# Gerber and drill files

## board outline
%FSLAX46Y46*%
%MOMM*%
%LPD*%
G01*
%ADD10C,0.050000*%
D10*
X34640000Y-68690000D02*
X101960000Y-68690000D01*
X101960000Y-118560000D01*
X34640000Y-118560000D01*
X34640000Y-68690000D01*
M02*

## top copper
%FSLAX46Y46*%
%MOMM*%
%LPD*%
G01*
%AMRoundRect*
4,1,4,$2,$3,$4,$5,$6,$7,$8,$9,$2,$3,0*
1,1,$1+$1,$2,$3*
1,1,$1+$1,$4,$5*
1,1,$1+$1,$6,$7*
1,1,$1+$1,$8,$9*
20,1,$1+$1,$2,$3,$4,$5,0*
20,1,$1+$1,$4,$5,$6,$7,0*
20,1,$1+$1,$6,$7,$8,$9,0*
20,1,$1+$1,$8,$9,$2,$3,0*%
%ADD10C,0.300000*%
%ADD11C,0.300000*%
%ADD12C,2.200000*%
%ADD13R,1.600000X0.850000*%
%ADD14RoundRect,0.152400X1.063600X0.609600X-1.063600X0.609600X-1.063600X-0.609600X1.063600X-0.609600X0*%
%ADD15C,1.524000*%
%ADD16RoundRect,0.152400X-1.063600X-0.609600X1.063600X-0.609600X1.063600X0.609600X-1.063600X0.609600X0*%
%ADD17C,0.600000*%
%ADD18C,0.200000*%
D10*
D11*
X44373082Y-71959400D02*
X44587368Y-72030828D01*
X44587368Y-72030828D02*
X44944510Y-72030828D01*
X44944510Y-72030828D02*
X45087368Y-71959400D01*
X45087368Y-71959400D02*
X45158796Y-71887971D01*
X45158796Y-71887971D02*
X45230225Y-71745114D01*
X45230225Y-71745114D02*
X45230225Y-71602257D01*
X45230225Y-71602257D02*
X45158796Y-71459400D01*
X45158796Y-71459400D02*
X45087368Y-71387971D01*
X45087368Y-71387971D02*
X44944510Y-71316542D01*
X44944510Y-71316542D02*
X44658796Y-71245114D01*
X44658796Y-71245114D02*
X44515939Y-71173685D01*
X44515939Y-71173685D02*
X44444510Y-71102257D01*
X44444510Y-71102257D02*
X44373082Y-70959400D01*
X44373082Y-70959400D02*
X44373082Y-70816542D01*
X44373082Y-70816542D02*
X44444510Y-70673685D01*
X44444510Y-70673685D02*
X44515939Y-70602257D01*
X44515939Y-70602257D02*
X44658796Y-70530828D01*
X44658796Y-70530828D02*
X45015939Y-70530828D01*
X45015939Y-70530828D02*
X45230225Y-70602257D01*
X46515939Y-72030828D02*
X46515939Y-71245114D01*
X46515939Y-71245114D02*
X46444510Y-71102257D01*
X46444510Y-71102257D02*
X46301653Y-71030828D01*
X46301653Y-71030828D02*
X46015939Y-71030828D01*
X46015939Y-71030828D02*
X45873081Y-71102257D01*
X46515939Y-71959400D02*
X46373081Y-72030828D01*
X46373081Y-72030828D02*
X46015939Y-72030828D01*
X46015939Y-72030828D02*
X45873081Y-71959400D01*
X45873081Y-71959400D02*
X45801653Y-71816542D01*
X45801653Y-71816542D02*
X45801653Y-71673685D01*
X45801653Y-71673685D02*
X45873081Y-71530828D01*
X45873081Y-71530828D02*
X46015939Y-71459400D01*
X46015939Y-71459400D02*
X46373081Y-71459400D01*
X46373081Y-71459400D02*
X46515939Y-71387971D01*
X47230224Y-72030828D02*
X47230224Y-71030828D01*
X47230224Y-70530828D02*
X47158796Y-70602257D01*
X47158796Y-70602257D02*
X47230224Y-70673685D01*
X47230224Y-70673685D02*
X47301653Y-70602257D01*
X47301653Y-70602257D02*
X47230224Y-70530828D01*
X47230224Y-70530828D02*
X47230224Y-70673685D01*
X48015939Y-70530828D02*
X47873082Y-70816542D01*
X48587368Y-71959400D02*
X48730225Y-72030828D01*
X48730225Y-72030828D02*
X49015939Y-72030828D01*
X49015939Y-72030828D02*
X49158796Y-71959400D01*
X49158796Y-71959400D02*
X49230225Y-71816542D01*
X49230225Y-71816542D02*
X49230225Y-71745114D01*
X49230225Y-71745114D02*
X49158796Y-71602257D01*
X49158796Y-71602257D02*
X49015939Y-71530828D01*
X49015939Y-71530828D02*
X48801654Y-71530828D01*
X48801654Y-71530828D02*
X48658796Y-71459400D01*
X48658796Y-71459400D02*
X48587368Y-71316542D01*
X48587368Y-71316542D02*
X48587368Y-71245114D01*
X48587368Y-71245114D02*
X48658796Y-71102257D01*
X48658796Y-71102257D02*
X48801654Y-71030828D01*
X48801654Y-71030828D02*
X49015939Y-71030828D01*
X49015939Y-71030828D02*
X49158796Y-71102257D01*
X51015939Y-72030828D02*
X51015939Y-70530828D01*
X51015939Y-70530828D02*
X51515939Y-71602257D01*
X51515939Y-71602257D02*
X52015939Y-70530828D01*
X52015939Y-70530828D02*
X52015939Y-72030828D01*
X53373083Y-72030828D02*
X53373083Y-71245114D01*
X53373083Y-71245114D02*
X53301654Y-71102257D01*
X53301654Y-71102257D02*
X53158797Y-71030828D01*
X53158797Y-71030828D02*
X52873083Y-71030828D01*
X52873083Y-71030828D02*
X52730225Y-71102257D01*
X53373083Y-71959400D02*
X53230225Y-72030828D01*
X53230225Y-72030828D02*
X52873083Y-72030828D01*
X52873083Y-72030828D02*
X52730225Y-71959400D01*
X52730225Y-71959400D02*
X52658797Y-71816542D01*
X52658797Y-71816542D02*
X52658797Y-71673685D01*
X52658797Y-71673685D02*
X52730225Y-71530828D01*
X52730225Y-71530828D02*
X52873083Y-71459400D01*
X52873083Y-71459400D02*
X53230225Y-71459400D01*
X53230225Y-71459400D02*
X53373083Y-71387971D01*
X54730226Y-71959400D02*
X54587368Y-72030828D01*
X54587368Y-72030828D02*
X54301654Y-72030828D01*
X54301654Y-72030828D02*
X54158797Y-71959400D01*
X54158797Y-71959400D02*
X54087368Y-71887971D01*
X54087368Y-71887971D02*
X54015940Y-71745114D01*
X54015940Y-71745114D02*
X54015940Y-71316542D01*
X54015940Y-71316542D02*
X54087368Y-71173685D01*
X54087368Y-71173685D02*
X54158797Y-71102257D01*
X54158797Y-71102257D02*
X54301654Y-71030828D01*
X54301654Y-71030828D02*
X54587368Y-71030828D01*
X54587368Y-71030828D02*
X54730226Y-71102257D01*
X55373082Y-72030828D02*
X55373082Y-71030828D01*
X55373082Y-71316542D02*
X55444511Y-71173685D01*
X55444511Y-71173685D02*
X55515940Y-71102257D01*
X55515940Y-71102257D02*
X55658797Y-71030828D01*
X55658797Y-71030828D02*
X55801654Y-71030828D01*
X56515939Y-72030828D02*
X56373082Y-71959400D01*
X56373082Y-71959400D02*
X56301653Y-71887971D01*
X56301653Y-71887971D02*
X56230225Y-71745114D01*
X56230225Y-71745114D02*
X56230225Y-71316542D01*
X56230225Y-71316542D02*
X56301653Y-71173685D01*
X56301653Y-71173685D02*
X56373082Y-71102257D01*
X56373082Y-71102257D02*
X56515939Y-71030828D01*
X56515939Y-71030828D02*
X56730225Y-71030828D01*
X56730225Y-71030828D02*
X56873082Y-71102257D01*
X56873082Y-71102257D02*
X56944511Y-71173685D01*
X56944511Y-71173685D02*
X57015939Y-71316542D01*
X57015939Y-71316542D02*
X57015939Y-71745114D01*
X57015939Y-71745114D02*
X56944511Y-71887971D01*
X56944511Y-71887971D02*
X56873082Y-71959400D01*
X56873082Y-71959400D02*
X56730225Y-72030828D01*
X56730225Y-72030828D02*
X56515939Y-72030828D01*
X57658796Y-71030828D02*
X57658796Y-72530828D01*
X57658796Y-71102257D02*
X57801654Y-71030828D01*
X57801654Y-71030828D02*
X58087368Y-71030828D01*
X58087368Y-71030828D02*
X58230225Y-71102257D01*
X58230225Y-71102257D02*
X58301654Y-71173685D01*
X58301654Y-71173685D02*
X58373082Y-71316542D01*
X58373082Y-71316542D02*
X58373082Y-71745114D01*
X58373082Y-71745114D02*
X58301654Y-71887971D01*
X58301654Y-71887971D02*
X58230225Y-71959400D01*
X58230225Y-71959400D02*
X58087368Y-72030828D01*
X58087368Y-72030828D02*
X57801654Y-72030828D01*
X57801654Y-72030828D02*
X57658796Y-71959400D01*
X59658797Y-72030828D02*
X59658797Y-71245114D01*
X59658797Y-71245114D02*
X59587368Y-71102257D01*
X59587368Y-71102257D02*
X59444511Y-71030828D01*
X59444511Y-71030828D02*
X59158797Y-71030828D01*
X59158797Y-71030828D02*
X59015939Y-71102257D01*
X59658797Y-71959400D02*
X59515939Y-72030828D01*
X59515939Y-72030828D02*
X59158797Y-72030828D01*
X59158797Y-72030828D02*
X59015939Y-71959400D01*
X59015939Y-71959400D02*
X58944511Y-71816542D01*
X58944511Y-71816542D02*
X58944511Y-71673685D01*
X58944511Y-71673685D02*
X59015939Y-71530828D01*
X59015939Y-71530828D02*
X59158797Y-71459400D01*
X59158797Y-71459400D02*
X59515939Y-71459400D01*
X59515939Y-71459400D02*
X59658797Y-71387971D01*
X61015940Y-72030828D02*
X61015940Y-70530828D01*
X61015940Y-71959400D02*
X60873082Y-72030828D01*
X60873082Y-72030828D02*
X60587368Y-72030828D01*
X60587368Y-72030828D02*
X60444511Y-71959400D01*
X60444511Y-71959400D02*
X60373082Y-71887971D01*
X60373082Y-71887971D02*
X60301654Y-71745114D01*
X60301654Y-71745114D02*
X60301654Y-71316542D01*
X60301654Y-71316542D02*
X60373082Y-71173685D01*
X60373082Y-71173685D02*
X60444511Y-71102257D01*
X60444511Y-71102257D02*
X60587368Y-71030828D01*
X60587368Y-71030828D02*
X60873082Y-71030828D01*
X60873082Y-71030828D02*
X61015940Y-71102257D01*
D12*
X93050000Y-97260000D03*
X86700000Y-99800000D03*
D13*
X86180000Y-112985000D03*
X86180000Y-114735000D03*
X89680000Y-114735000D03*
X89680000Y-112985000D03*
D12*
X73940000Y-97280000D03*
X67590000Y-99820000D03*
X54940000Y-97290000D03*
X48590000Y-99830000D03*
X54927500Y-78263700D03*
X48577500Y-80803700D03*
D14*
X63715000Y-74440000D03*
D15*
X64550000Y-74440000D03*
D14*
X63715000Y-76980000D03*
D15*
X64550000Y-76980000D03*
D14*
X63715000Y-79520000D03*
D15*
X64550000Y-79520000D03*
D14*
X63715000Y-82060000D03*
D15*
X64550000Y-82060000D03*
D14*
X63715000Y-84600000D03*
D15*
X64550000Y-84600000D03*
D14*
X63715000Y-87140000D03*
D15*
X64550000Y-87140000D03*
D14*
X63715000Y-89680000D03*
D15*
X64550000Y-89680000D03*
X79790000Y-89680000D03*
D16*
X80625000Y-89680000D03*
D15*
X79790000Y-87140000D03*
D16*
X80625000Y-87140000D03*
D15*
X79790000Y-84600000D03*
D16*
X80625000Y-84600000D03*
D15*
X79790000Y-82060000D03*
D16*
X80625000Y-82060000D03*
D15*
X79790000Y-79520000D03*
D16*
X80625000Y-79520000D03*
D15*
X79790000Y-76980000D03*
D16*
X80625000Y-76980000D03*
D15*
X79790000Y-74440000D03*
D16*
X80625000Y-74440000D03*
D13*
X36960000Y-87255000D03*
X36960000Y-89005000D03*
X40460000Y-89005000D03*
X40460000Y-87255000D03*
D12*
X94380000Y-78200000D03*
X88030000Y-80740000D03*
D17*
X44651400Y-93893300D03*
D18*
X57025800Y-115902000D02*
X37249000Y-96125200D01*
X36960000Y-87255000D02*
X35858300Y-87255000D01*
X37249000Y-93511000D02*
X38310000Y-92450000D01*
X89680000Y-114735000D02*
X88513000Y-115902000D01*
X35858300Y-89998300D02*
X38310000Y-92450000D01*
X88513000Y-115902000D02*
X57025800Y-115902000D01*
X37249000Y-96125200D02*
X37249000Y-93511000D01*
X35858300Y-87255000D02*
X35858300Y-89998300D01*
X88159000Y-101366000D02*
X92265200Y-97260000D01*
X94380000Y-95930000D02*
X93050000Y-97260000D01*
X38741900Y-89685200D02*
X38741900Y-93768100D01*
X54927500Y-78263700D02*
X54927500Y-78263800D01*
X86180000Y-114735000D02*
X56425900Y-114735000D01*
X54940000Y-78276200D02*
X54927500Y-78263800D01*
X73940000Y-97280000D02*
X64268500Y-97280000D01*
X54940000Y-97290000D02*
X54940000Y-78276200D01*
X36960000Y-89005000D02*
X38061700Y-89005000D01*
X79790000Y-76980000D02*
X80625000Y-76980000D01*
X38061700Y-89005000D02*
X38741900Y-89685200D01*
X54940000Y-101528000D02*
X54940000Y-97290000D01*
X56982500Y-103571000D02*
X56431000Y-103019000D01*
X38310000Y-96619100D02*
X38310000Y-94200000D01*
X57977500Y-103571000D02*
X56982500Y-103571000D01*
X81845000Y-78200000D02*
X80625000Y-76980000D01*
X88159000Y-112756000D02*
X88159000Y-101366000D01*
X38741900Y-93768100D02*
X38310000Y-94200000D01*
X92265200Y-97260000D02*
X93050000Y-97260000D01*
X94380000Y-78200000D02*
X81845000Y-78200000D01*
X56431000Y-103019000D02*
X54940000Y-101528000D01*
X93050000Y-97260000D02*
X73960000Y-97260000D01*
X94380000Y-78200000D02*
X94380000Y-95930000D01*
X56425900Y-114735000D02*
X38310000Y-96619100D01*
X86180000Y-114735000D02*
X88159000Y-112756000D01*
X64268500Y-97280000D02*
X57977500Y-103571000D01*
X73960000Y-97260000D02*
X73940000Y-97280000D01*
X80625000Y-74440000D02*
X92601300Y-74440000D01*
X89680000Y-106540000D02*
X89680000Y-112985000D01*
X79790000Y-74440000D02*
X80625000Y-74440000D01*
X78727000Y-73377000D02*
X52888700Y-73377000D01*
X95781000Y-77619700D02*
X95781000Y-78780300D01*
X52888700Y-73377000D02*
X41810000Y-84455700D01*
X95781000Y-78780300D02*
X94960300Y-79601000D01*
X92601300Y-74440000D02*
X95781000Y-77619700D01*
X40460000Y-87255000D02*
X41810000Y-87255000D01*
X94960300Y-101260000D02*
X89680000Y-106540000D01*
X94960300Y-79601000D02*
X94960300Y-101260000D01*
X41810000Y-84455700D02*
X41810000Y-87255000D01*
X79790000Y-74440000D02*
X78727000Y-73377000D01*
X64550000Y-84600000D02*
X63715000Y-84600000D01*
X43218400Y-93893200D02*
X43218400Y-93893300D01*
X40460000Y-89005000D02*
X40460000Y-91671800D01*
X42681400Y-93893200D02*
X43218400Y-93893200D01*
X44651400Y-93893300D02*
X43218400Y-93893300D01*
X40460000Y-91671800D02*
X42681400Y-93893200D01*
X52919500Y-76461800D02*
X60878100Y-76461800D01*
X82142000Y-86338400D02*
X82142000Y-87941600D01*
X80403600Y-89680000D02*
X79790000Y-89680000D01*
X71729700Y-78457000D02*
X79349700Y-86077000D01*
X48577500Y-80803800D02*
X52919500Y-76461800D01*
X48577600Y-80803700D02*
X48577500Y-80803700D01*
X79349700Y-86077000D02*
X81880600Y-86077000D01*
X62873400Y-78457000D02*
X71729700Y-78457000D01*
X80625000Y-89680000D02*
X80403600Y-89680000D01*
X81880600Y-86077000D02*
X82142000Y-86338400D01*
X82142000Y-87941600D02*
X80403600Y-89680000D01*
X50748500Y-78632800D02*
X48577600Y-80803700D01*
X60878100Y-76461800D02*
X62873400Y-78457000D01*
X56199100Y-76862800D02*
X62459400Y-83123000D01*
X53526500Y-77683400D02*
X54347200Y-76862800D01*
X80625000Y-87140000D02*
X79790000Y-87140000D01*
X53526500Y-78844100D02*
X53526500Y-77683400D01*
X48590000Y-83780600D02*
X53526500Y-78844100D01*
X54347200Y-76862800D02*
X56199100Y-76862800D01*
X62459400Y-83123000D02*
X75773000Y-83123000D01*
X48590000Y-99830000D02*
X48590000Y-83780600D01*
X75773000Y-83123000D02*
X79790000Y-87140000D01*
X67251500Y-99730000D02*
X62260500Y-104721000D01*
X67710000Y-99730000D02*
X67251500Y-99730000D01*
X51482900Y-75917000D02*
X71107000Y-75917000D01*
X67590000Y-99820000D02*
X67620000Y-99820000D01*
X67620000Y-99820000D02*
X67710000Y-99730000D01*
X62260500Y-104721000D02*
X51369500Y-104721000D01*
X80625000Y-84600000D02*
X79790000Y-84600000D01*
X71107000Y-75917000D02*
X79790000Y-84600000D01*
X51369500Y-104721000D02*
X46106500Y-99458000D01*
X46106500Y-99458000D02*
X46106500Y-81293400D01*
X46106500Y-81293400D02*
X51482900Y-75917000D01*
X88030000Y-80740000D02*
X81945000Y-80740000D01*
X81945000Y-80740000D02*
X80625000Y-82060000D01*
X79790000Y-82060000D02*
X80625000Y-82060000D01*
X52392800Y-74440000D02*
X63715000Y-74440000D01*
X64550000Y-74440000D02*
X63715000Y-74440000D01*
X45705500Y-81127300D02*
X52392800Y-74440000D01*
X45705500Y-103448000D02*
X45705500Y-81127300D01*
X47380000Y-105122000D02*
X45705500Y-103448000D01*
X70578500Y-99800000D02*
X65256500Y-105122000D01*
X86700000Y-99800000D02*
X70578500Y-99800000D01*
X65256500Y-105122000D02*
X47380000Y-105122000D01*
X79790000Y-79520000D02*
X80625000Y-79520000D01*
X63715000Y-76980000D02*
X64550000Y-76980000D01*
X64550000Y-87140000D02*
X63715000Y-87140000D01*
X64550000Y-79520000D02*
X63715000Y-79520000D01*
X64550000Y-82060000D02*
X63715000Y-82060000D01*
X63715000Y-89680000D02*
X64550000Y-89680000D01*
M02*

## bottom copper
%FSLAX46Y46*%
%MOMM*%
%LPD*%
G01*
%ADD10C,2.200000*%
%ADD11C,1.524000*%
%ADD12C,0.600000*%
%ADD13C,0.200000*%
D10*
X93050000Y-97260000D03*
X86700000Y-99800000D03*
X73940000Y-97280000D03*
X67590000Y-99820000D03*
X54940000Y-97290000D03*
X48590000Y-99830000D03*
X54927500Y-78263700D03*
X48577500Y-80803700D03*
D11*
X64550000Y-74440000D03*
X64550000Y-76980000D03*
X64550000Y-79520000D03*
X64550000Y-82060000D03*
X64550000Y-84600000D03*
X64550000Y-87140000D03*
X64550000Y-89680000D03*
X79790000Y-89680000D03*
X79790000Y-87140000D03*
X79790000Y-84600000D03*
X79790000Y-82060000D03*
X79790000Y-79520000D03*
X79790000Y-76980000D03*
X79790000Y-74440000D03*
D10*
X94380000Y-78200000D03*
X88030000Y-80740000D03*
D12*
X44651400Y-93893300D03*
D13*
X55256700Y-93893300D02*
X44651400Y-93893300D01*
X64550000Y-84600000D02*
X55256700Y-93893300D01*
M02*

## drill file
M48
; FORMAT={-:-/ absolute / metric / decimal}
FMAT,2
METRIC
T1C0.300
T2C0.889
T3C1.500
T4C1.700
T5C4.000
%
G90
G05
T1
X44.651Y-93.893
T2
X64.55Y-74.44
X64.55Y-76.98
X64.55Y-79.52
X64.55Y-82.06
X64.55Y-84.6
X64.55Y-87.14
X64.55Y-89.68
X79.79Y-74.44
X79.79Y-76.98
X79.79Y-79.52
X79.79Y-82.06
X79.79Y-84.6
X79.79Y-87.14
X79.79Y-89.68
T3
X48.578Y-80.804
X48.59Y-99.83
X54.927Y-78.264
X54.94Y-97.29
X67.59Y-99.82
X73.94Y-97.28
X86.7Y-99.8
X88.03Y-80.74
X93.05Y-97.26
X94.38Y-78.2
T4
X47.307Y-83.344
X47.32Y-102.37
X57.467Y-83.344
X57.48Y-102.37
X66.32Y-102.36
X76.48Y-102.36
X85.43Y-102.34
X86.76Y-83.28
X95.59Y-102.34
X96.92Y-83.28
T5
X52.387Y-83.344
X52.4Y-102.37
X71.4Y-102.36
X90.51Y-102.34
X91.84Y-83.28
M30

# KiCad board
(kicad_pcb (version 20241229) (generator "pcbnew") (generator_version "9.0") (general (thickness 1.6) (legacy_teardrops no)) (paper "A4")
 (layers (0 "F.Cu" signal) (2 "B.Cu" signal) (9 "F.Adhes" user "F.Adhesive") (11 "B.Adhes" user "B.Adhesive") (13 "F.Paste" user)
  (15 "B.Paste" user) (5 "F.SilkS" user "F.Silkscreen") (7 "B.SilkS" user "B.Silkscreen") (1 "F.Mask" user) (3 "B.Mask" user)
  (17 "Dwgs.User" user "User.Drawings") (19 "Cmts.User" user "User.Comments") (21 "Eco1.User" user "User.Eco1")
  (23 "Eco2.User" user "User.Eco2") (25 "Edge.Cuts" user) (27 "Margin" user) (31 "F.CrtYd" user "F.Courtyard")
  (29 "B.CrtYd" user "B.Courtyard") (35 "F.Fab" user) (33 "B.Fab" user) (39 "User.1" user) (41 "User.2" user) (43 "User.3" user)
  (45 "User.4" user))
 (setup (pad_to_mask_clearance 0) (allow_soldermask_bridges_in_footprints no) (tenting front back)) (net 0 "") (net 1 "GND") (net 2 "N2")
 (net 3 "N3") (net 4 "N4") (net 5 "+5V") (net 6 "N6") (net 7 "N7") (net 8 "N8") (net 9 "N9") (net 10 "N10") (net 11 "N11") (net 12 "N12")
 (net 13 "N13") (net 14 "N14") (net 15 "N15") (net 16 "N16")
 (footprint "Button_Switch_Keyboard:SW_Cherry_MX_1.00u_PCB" (layer "F.Cu") (at 93.05 97.26)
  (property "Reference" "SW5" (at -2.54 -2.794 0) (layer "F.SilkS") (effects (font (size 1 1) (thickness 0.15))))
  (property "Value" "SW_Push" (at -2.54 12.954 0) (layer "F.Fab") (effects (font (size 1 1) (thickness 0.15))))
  (pad "" np_thru_hole circle (at -7.62 5.08) (size 1.7 1.7) (drill 1.7) (layers "*.Cu" "*.Mask"))
  (pad "" np_thru_hole circle (at -2.54 5.08) (size 4 4) (drill 4) (layers "*.Cu" "*.Mask"))
  (pad "" np_thru_hole circle (at 2.54 5.08) (size 1.7 1.7) (drill 1.7) (layers "*.Cu" "*.Mask"))
  (pad "1" thru_hole circle (at 0 0) (size 2.2 2.2) (drill 1.5) (layers "*.Cu" "*.Mask") (remove_unused_layers no) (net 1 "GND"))
  (pad "2" thru_hole circle (at -6.35 2.54) (size 2.2 2.2) (drill 1.5) (layers "*.Cu" "*.Mask") (remove_unused_layers no) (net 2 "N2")))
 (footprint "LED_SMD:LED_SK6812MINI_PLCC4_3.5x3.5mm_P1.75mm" (layer "F.Cu") (at 87.93 113.86)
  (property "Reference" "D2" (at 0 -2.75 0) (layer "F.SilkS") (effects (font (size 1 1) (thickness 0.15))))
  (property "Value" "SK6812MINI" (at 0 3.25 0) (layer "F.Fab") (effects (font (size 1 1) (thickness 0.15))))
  (pad "1" smd rect (at -1.75 -0.875) (size 1.6 0.85) (layers "F.Cu" "F.Mask" "F.Paste") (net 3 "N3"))
  (pad "2" smd rect (at -1.75 0.875) (size 1.6 0.85) (layers "F.Cu" "F.Mask" "F.Paste") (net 1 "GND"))
  (pad "3" smd rect (at 1.75 0.875) (size 1.6 0.85) (layers "F.Cu" "F.Mask" "F.Paste") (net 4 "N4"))
  (pad "4" smd rect (at 1.75 -0.875) (size 1.6 0.85) (layers "F.Cu" "F.Mask" "F.Paste") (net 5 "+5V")))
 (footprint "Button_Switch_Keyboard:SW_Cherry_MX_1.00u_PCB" (layer "F.Cu") (at 73.94 97.28)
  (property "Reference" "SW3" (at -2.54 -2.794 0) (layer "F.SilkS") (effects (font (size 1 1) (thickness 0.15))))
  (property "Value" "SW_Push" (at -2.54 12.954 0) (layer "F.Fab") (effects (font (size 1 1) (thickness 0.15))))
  (pad "" np_thru_hole circle (at -7.62 5.08) (size 1.7 1.7) (drill 1.7) (layers "*.Cu" "*.Mask"))
  (pad "" np_thru_hole circle (at -2.54 5.08) (size 4 4) (drill 4) (layers "*.Cu" "*.Mask"))
  (pad "" np_thru_hole circle (at 2.54 5.08) (size 1.7 1.7) (drill 1.7) (layers "*.Cu" "*.Mask"))
  (pad "1" thru_hole circle (at 0 0) (size 2.2 2.2) (drill 1.5) (layers "*.Cu" "*.Mask") (remove_unused_layers no) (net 1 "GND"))
  (pad "2" thru_hole circle (at -6.35 2.54) (size 2.2 2.2) (drill 1.5) (layers "*.Cu" "*.Mask") (remove_unused_layers no) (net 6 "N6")))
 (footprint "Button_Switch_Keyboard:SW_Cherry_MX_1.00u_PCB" (layer "F.Cu") (at 54.94 97.29)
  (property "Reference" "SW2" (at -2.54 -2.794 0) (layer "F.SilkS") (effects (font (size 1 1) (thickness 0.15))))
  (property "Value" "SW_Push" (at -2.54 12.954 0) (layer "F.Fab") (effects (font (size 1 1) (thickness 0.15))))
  (pad "" np_thru_hole circle (at -7.62 5.08) (size 1.7 1.7) (drill 1.7) (layers "*.Cu" "*.Mask"))
  (pad "" np_thru_hole circle (at -2.54 5.08) (size 4 4) (drill 4) (layers "*.Cu" "*.Mask"))
  (pad "" np_thru_hole circle (at 2.54 5.08) (size 1.7 1.7) (drill 1.7) (layers "*.Cu" "*.Mask"))
  (pad "1" thru_hole circle (at 0 0) (size 2.2 2.2) (drill 1.5) (layers "*.Cu" "*.Mask") (remove_unused_layers no) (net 1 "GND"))
  (pad "2" thru_hole circle (at -6.35 2.54) (size 2.2 2.2) (drill 1.5) (layers "*.Cu" "*.Mask") (remove_unused_layers no) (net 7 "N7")))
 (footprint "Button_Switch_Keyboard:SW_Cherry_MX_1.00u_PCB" (layer "F.Cu") (at 54.9275 78.2637)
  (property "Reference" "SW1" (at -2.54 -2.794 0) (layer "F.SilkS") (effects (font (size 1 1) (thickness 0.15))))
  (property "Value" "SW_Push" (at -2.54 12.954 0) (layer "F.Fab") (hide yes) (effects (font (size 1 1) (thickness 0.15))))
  (pad "" np_thru_hole circle (at -7.62 5.08) (size 1.7 1.7) (drill 1.7) (layers "*.Cu" "*.Mask"))
  (pad "" np_thru_hole circle (at -2.54 5.08) (size 4 4) (drill 4) (layers "*.Cu" "*.Mask"))
  (pad "" np_thru_hole circle (at 2.54 5.08) (size 1.7 1.7) (drill 1.7) (layers "*.Cu" "*.Mask"))
  (pad "1" thru_hole circle (at 0 0) (size 2.2 2.2) (drill 1.5) (layers "*.Cu" "*.Mask") (remove_unused_layers no) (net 1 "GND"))
  (pad "2" thru_hole circle (at -6.35 2.54) (size 2.2 2.2) (drill 1.5) (layers "*.Cu" "*.Mask") (remove_unused_layers no) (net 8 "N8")))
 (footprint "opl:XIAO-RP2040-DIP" (layer "F.Cu") (at 72.17 82.06)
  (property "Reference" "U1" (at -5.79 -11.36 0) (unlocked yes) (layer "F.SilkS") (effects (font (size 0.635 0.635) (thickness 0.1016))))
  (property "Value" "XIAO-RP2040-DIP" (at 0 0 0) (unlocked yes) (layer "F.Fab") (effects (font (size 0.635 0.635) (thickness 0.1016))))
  (pad "1" smd roundrect (at -8.455 -7.62 180) (size 2.432 1.524) (layers "F.Cu" "F.Mask") (roundrect_rratio 0.1) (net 2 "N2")
   (thermal_bridge_angle 45))
  (pad "1" thru_hole circle (at -7.62 -7.62 180) (size 1.524 1.524) (drill 0.889) (layers "*.Cu" "*.Mask") (remove_unused_layers no)
   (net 2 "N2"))
  (pad "2" smd roundrect (at -8.455 -5.08 180) (size 2.432 1.524) (layers "F.Cu" "F.Mask") (roundrect_rratio 0.1) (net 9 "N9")
   (thermal_bridge_angle 45))
  (pad "2" thru_hole circle (at -7.62 -5.08 180) (size 1.524 1.524) (drill 0.889) (layers "*.Cu" "*.Mask") (remove_unused_layers no)
   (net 9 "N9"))
  (pad "3" smd roundrect (at -8.455 -2.54 180) (size 2.432 1.524) (layers "F.Cu" "F.Mask") (roundrect_rratio 0.1) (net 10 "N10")
   (thermal_bridge_angle 45))
  (pad "3" thru_hole circle (at -7.62 -2.54 180) (size 1.524 1.524) (drill 0.889) (layers "*.Cu" "*.Mask") (remove_unused_layers no)
   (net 10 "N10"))
  (pad "4" smd roundrect (at -8.455 0 180) (size 2.432 1.524) (layers "F.Cu" "F.Mask") (roundrect_rratio 0.1) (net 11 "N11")
   (thermal_bridge_angle 45))
  (pad "4" thru_hole circle (at -7.62 0 180) (size 1.524 1.524) (drill 0.889) (layers "*.Cu" "*.Mask") (remove_unused_layers no)
   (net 11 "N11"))
  (pad "5" smd roundrect (at -8.455 2.54 180) (size 2.432 1.524) (layers "F.Cu" "F.Mask") (roundrect_rratio 0.1) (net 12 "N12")
   (thermal_bridge_angle 45))
  (pad "5" thru_hole circle (at -7.62 2.54 180) (size 1.524 1.524) (drill 0.889) (layers "*.Cu" "*.Mask") (remove_unused_layers no)
   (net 12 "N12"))
  (pad "6" smd roundrect (at -8.455 5.08 180) (size 2.432 1.524) (layers "F.Cu" "F.Mask") (roundrect_rratio 0.1) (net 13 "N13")
   (thermal_bridge_angle 45))
  (pad "6" thru_hole circle (at -7.62 5.08 180) (size 1.524 1.524) (drill 0.889) (layers "*.Cu" "*.Mask") (remove_unused_layers no)
   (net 13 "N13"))
  (pad "7" smd roundrect (at -8.455 7.62 180) (size 2.432 1.524) (layers "F.Cu" "F.Mask") (roundrect_rratio 0.1) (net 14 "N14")
   (thermal_bridge_angle 45))
  (pad "7" thru_hole circle (at -7.62 7.62 180) (size 1.524 1.524) (drill 0.889) (layers "*.Cu" "*.Mask") (remove_unused_layers no)
   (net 14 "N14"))
  (pad "8" thru_hole circle (at 7.62 7.62) (size 1.524 1.524) (drill 0.889) (layers "*.Cu" "*.Mask") (remove_unused_layers no) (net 8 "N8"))
  (pad "8" smd roundrect (at 8.455 7.62) (size 2.432 1.524) (layers "F.Cu" "F.Mask") (roundrect_rratio 0.1) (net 8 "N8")
   (thermal_bridge_angle 45))
  (pad "9" thru_hole circle (at 7.62 5.08) (size 1.524 1.524) (drill 0.889) (layers "*.Cu" "*.Mask") (remove_unused_layers no) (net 7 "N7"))
  (pad "9" smd roundrect (at 8.455 5.08) (size 2.432 1.524) (layers "F.Cu" "F.Mask") (roundrect_rratio 0.1) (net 7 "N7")
   (thermal_bridge_angle 45))
  (pad "10" thru_hole circle (at 7.62 2.54) (size 1.524 1.524) (drill 0.889) (layers "*.Cu" "*.Mask") (remove_unused_layers no) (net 6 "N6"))
  (pad "10" smd roundrect (at 8.455 2.54) (size 2.432 1.524) (layers "F.Cu" "F.Mask") (roundrect_rratio 0.1) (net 6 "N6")
   (thermal_bridge_angle 45))
  (pad "11" thru_hole circle (at 7.62 0) (size 1.524 1.524) (drill 0.889) (layers "*.Cu" "*.Mask") (remove_unused_layers no) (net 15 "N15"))
  (pad "11" smd roundrect (at 8.455 0) (size 2.432 1.524) (layers "F.Cu" "F.Mask") (roundrect_rratio 0.1) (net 15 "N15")
   (thermal_bridge_angle 45))
  (pad "12" thru_hole circle (at 7.62 -2.54) (size 1.524 1.524) (drill 0.889) (layers "*.Cu" "*.Mask") (remove_unused_layers no)
   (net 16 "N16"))
  (pad "12" smd roundrect (at 8.455 -2.54) (size 2.432 1.524) (layers "F.Cu" "F.Mask") (roundrect_rratio 0.1) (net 16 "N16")
   (thermal_bridge_angle 45))
  (pad "13" thru_hole circle (at 7.62 -5.08) (size 1.524 1.524) (drill 0.889) (layers "*.Cu" "*.Mask") (remove_unused_layers no)
   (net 1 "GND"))
  (pad "13" smd roundrect (at 8.455 -5.08) (size 2.432 1.524) (layers "F.Cu" "F.Mask") (roundrect_rratio 0.1) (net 1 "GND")
   (thermal_bridge_angle 45))
  (pad "14" thru_hole circle (at 7.62 -7.62) (size 1.524 1.524) (drill 0.889) (layers "*.Cu" "*.Mask") (remove_unused_layers no)
   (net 5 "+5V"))
  (pad "14" smd roundrect (at 8.455 -7.62) (size 2.432 1.524) (layers "F.Cu" "F.Mask") (roundrect_rratio 0.1) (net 5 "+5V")
   (thermal_bridge_angle 45)))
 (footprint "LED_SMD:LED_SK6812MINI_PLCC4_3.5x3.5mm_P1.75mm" (layer "F.Cu") (at 38.71 88.13)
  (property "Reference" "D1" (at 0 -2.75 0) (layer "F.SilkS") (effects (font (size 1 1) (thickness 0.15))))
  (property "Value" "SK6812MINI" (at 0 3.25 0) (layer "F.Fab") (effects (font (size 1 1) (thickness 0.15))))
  (pad "1" smd rect (at -1.75 -0.875) (size 1.6 0.85) (layers "F.Cu" "F.Mask" "F.Paste") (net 4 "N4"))
  (pad "2" smd rect (at -1.75 0.875) (size 1.6 0.85) (layers "F.Cu" "F.Mask" "F.Paste") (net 1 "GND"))
  (pad "3" smd rect (at 1.75 0.875) (size 1.6 0.85) (layers "F.Cu" "F.Mask" "F.Paste") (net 12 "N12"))
  (pad "4" smd rect (at 1.75 -0.875) (size 1.6 0.85) (layers "F.Cu" "F.Mask" "F.Paste") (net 5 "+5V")))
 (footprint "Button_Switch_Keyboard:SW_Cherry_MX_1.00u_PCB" (layer "F.Cu") (at 94.38 78.2)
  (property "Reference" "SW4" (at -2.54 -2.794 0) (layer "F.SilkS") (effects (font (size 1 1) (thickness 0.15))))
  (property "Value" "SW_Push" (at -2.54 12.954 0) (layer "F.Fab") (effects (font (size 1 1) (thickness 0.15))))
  (pad "" np_thru_hole circle (at -7.62 5.08) (size 1.7 1.7) (drill 1.7) (layers "*.Cu" "*.Mask"))
  (pad "" np_thru_hole circle (at -2.54 5.08) (size 4 4) (drill 4) (layers "*.Cu" "*.Mask"))
  (pad "" np_thru_hole circle (at 2.54 5.08) (size 1.7 1.7) (drill 1.7) (layers "*.Cu" "*.Mask"))
  (pad "1" thru_hole circle (at 0 0) (size 2.2 2.2) (drill 1.5) (layers "*.Cu" "*.Mask") (remove_unused_layers no) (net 1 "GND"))
  (pad "2" thru_hole circle (at -6.35 2.54) (size 2.2 2.2) (drill 1.5) (layers "*.Cu" "*.Mask") (remove_unused_layers no) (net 15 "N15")))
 (gr_rect (start 34.64 68.69) (end 101.96 118.56) (stroke (width 0.05) (type default)) (fill no) (layer "Edge.Cuts"))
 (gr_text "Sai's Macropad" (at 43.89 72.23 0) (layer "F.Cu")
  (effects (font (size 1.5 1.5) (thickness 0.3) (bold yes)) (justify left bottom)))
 (segment (start 57.0258 115.902) (end 37.249 96.1252) (width 0.2) (layer "F.Cu") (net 4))
 (segment (start 36.96 87.255) (end 35.8583 87.255) (width 0.2) (layer "F.Cu") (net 4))
 (segment (start 37.249 93.511) (end 38.31 92.45) (width 0.2) (layer "F.Cu") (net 4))
 (segment (start 89.68 114.735) (end 88.513 115.902) (width 0.2) (layer "F.Cu") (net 4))
 (segment (start 35.8583 89.9983) (end 38.31 92.45) (width 0.2) (layer "F.Cu") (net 4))
 (segment (start 88.513 115.902) (end 57.0258 115.902) (width 0.2) (layer "F.Cu") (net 4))
 (segment (start 37.249 96.1252) (end 37.249 93.511) (width 0.2) (layer "F.Cu") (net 4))
 (segment (start 35.8583 87.255) (end 35.8583 89.9983) (width 0.2) (layer "F.Cu") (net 4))
 (segment (start 88.159 101.366) (end 92.2652 97.26) (width 0.2) (layer "F.Cu") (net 1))
 (segment (start 94.38 95.93) (end 93.05 97.26) (width 0.2) (layer "F.Cu") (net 1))
 (segment (start 38.7419 89.6852) (end 38.7419 93.7681) (width 0.2) (layer "F.Cu") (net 1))
 (segment (start 54.9275 78.2637) (end 54.9275 78.2638) (width 0.2) (layer "F.Cu") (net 1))
 (segment (start 86.18 114.735) (end 56.4259 114.735) (width 0.2) (layer "F.Cu") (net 1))
 (segment (start 54.94 78.2762) (end 54.9275 78.2638) (width 0.2) (layer "F.Cu") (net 1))
 (segment (start 73.94 97.28) (end 64.2685 97.28) (width 0.2) (layer "F.Cu") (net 1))
 (segment (start 54.94 97.29) (end 54.94 78.2762) (width 0.2) (layer "F.Cu") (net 1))
 (segment (start 36.96 89.005) (end 38.0617 89.005) (width 0.2) (layer "F.Cu") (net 1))
 (segment (start 79.79 76.98) (end 80.625 76.98) (width 0.2) (layer "F.Cu") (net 1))
 (segment (start 38.0617 89.005) (end 38.7419 89.6852) (width 0.2) (layer "F.Cu") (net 1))
 (segment (start 54.94 101.528) (end 54.94 97.29) (width 0.2) (layer "F.Cu") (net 1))
 (segment (start 56.9825 103.571) (end 56.431 103.019) (width 0.2) (layer "F.Cu") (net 1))
 (segment (start 38.31 96.6191) (end 38.31 94.2) (width 0.2) (layer "F.Cu") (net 1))
 (segment (start 57.9775 103.571) (end 56.9825 103.571) (width 0.2) (layer "F.Cu") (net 1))
 (segment (start 81.845 78.2) (end 80.625 76.98) (width 0.2) (layer "F.Cu") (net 1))
 (segment (start 88.159 112.756) (end 88.159 101.366) (width 0.2) (layer "F.Cu") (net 1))
 (segment (start 38.7419 93.7681) (end 38.31 94.2) (width 0.2) (layer "F.Cu") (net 1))
 (segment (start 92.2652 97.26) (end 93.05 97.26) (width 0.2) (layer "F.Cu") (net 1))
 (segment (start 94.38 78.2) (end 81.845 78.2) (width 0.2) (layer "F.Cu") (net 1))
 (segment (start 56.431 103.019) (end 54.94 101.528) (width 0.2) (layer "F.Cu") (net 1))
 (segment (start 93.05 97.26) (end 73.96 97.26) (width 0.2) (layer "F.Cu") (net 1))
 (segment (start 94.38 78.2) (end 94.38 95.93) (width 0.2) (layer "F.Cu") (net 1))
 (segment (start 56.4259 114.735) (end 38.31 96.6191) (width 0.2) (layer "F.Cu") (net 1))
 (segment (start 86.18 114.735) (end 88.159 112.756) (width 0.2) (layer "F.Cu") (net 1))
 (segment (start 64.2685 97.28) (end 57.9775 103.571) (width 0.2) (layer "F.Cu") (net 1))
 (segment (start 73.96 97.26) (end 73.94 97.28) (width 0.2) (layer "F.Cu") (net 1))
 (segment (start 80.625 74.44) (end 92.6013 74.44) (width 0.2) (layer "F.Cu") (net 5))
 (segment (start 89.68 106.54) (end 89.68 112.985) (width 0.2) (layer "F.Cu") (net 5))
 (segment (start 79.79 74.44) (end 80.625 74.44) (width 0.2) (layer "F.Cu") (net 5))
 (segment (start 78.727 73.377) (end 52.8887 73.377) (width 0.2) (layer "F.Cu") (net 5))
 (segment (start 95.781 77.6197) (end 95.781 78.7803) (width 0.2) (layer "F.Cu") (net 5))
 (segment (start 52.8887 73.377) (end 41.81 84.4557) (width 0.2) (layer "F.Cu") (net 5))
 (segment (start 95.781 78.7803) (end 94.9603 79.601) (width 0.2) (layer "F.Cu") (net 5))
 (segment (start 92.6013 74.44) (end 95.781 77.6197) (width 0.2) (layer "F.Cu") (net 5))
 (segment (start 40.46 87.255) (end 41.81 87.255) (width 0.2) (layer "F.Cu") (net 5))
 (segment (start 94.9603 101.26) (end 89.68 106.54) (width 0.2) (layer "F.Cu") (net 5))
 (segment (start 94.9603 79.601) (end 94.9603 101.26) (width 0.2) (layer "F.Cu") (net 5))
 (segment (start 41.81 84.4557) (end 41.81 87.255) (width 0.2) (layer "F.Cu") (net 5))
 (segment (start 79.79 74.44) (end 78.727 73.377) (width 0.2) (layer "F.Cu") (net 5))
 (segment (start 64.55 84.6) (end 63.715 84.6) (width 0.2) (layer "F.Cu") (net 12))
 (segment (start 43.2184 93.8932) (end 43.2184 93.8933) (width 0.2) (layer "F.Cu") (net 12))
 (segment (start 40.46 89.005) (end 40.46 91.6718) (width 0.2) (layer "F.Cu") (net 12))
 (segment (start 42.6814 93.8932) (end 43.2184 93.8932) (width 0.2) (layer "F.Cu") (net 12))
 (segment (start 44.6514 93.8933) (end 43.2184 93.8933) (width 0.2) (layer "F.Cu") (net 12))
 (segment (start 40.46 91.6718) (end 42.6814 93.8932) (width 0.2) (layer "F.Cu") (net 12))
 (via (at 44.6514 93.8933) (size 0.6) (drill 0.3) (layers "F.Cu" "B.Cu") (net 12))
 (segment (start 55.2567 93.8933) (end 44.6514 93.8933) (width 0.2) (layer "B.Cu") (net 12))
 (segment (start 64.55 84.6) (end 55.2567 93.8933) (width 0.2) (layer "B.Cu") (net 12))
 (segment (start 52.9195 76.4618) (end 60.8781 76.4618) (width 0.2) (layer "F.Cu") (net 8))
 (segment (start 82.142 86.3384) (end 82.142 87.9416) (width 0.2) (layer "F.Cu") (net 8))
 (segment (start 80.4036 89.68) (end 79.79 89.68) (width 0.2) (layer "F.Cu") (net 8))
 (segment (start 71.7297 78.457) (end 79.3497 86.077) (width 0.2) (layer "F.Cu") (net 8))
 (segment (start 48.5775 80.8038) (end 52.9195 76.4618) (width 0.2) (layer "F.Cu") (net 8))
 (segment (start 48.5776 80.8037) (end 48.5775 80.8037) (width 0.2) (layer "F.Cu") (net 8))
 (segment (start 79.3497 86.077) (end 81.8806 86.077) (width 0.2) (layer "F.Cu") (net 8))
 (segment (start 62.8734 78.457) (end 71.7297 78.457) (width 0.2) (layer "F.Cu") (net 8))
 (segment (start 80.625 89.68) (end 80.4036 89.68) (width 0.2) (layer "F.Cu") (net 8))
 (segment (start 81.8806 86.077) (end 82.142 86.3384) (width 0.2) (layer "F.Cu") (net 8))
 (segment (start 82.142 87.9416) (end 80.4036 89.68) (width 0.2) (layer "F.Cu") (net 8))
 (segment (start 50.7485 78.6328) (end 48.5776 80.8037) (width 0.2) (layer "F.Cu") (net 8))
 (segment (start 60.8781 76.4618) (end 62.8734 78.457) (width 0.2) (layer "F.Cu") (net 8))
 (segment (start 56.1991 76.8628) (end 62.4594 83.123) (width 0.2) (layer "F.Cu") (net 7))
 (segment (start 53.5265 77.6834) (end 54.3472 76.8628) (width 0.2) (layer "F.Cu") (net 7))
 (segment (start 80.625 87.14) (end 79.79 87.14) (width 0.2) (layer "F.Cu") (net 7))
 (segment (start 53.5265 78.8441) (end 53.5265 77.6834) (width 0.2) (layer "F.Cu") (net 7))
 (segment (start 48.59 83.7806) (end 53.5265 78.8441) (width 0.2) (layer "F.Cu") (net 7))
 (segment (start 54.3472 76.8628) (end 56.1991 76.8628) (width 0.2) (layer "F.Cu") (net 7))
 (segment (start 62.4594 83.123) (end 75.773 83.123) (width 0.2) (layer "F.Cu") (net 7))
 (segment (start 48.59 99.83) (end 48.59 83.7806) (width 0.2) (layer "F.Cu") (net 7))
 (segment (start 75.773 83.123) (end 79.79 87.14) (width 0.2) (layer "F.Cu") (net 7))
 (segment (start 67.2515 99.73) (end 62.2605 104.721) (width 0.2) (layer "F.Cu") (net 6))
 (segment (start 67.71 99.73) (end 67.2515 99.73) (width 0.2) (layer "F.Cu") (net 6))
 (segment (start 51.4829 75.917) (end 71.107 75.917) (width 0.2) (layer "F.Cu") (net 6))
 (segment (start 67.59 99.82) (end 67.62 99.82) (width 0.2) (layer "F.Cu") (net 6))
 (segment (start 67.62 99.82) (end 67.71 99.73) (width 0.2) (layer "F.Cu") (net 6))
 (segment (start 62.2605 104.721) (end 51.3695 104.721) (width 0.2) (layer "F.Cu") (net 6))
 (segment (start 80.625 84.6) (end 79.79 84.6) (width 0.2) (layer "F.Cu") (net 6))
 (segment (start 71.107 75.917) (end 79.79 84.6) (width 0.2) (layer "F.Cu") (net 6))
 (segment (start 51.3695 104.721) (end 46.1065 99.458) (width 0.2) (layer "F.Cu") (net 6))
 (segment (start 46.1065 99.458) (end 46.1065 81.2934) (width 0.2) (layer "F.Cu") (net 6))
 (segment (start 46.1065 81.2934) (end 51.4829 75.917) (width 0.2) (layer "F.Cu") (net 6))
 (segment (start 88.03 80.74) (end 81.945 80.74) (width 0.2) (layer "F.Cu") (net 15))
 (segment (start 81.945 80.74) (end 80.625 82.06) (width 0.2) (layer "F.Cu") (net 15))
 (segment (start 79.79 82.06) (end 80.625 82.06) (width 0.2) (layer "F.Cu") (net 15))
 (segment (start 52.3928 74.44) (end 63.715 74.44) (width 0.2) (layer "F.Cu") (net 2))
 (segment (start 64.55 74.44) (end 63.715 74.44) (width 0.2) (layer "F.Cu") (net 2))
 (segment (start 45.7055 81.1273) (end 52.3928 74.44) (width 0.2) (layer "F.Cu") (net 2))
 (segment (start 45.7055 103.448) (end 45.7055 81.1273) (width 0.2) (layer "F.Cu") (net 2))
 (segment (start 47.38 105.122) (end 45.7055 103.448) (width 0.2) (layer "F.Cu") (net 2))
 (segment (start 70.5785 99.8) (end 65.2565 105.122) (width 0.2) (layer "F.Cu") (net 2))
 (segment (start 86.7 99.8) (end 70.5785 99.8) (width 0.2) (layer "F.Cu") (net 2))
 (segment (start 65.2565 105.122) (end 47.38 105.122) (width 0.2) (layer "F.Cu") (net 2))
 (segment (start 79.79 79.52) (end 80.625 79.52) (width 0.2) (layer "F.Cu") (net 16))
 (segment (start 63.715 76.98) (end 64.55 76.98) (width 0.2) (layer "F.Cu") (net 9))
 (segment (start 64.55 87.14) (end 63.715 87.14) (width 0.2) (layer "F.Cu") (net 13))
 (segment (start 64.55 79.52) (end 63.715 79.52) (width 0.2) (layer "F.Cu") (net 10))
 (segment (start 64.55 82.06) (end 63.715 82.06) (width 0.2) (layer "F.Cu") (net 11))
 (segment (start 63.715 89.68) (end 64.55 89.68) (width 0.2) (layer "F.Cu") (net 14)))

